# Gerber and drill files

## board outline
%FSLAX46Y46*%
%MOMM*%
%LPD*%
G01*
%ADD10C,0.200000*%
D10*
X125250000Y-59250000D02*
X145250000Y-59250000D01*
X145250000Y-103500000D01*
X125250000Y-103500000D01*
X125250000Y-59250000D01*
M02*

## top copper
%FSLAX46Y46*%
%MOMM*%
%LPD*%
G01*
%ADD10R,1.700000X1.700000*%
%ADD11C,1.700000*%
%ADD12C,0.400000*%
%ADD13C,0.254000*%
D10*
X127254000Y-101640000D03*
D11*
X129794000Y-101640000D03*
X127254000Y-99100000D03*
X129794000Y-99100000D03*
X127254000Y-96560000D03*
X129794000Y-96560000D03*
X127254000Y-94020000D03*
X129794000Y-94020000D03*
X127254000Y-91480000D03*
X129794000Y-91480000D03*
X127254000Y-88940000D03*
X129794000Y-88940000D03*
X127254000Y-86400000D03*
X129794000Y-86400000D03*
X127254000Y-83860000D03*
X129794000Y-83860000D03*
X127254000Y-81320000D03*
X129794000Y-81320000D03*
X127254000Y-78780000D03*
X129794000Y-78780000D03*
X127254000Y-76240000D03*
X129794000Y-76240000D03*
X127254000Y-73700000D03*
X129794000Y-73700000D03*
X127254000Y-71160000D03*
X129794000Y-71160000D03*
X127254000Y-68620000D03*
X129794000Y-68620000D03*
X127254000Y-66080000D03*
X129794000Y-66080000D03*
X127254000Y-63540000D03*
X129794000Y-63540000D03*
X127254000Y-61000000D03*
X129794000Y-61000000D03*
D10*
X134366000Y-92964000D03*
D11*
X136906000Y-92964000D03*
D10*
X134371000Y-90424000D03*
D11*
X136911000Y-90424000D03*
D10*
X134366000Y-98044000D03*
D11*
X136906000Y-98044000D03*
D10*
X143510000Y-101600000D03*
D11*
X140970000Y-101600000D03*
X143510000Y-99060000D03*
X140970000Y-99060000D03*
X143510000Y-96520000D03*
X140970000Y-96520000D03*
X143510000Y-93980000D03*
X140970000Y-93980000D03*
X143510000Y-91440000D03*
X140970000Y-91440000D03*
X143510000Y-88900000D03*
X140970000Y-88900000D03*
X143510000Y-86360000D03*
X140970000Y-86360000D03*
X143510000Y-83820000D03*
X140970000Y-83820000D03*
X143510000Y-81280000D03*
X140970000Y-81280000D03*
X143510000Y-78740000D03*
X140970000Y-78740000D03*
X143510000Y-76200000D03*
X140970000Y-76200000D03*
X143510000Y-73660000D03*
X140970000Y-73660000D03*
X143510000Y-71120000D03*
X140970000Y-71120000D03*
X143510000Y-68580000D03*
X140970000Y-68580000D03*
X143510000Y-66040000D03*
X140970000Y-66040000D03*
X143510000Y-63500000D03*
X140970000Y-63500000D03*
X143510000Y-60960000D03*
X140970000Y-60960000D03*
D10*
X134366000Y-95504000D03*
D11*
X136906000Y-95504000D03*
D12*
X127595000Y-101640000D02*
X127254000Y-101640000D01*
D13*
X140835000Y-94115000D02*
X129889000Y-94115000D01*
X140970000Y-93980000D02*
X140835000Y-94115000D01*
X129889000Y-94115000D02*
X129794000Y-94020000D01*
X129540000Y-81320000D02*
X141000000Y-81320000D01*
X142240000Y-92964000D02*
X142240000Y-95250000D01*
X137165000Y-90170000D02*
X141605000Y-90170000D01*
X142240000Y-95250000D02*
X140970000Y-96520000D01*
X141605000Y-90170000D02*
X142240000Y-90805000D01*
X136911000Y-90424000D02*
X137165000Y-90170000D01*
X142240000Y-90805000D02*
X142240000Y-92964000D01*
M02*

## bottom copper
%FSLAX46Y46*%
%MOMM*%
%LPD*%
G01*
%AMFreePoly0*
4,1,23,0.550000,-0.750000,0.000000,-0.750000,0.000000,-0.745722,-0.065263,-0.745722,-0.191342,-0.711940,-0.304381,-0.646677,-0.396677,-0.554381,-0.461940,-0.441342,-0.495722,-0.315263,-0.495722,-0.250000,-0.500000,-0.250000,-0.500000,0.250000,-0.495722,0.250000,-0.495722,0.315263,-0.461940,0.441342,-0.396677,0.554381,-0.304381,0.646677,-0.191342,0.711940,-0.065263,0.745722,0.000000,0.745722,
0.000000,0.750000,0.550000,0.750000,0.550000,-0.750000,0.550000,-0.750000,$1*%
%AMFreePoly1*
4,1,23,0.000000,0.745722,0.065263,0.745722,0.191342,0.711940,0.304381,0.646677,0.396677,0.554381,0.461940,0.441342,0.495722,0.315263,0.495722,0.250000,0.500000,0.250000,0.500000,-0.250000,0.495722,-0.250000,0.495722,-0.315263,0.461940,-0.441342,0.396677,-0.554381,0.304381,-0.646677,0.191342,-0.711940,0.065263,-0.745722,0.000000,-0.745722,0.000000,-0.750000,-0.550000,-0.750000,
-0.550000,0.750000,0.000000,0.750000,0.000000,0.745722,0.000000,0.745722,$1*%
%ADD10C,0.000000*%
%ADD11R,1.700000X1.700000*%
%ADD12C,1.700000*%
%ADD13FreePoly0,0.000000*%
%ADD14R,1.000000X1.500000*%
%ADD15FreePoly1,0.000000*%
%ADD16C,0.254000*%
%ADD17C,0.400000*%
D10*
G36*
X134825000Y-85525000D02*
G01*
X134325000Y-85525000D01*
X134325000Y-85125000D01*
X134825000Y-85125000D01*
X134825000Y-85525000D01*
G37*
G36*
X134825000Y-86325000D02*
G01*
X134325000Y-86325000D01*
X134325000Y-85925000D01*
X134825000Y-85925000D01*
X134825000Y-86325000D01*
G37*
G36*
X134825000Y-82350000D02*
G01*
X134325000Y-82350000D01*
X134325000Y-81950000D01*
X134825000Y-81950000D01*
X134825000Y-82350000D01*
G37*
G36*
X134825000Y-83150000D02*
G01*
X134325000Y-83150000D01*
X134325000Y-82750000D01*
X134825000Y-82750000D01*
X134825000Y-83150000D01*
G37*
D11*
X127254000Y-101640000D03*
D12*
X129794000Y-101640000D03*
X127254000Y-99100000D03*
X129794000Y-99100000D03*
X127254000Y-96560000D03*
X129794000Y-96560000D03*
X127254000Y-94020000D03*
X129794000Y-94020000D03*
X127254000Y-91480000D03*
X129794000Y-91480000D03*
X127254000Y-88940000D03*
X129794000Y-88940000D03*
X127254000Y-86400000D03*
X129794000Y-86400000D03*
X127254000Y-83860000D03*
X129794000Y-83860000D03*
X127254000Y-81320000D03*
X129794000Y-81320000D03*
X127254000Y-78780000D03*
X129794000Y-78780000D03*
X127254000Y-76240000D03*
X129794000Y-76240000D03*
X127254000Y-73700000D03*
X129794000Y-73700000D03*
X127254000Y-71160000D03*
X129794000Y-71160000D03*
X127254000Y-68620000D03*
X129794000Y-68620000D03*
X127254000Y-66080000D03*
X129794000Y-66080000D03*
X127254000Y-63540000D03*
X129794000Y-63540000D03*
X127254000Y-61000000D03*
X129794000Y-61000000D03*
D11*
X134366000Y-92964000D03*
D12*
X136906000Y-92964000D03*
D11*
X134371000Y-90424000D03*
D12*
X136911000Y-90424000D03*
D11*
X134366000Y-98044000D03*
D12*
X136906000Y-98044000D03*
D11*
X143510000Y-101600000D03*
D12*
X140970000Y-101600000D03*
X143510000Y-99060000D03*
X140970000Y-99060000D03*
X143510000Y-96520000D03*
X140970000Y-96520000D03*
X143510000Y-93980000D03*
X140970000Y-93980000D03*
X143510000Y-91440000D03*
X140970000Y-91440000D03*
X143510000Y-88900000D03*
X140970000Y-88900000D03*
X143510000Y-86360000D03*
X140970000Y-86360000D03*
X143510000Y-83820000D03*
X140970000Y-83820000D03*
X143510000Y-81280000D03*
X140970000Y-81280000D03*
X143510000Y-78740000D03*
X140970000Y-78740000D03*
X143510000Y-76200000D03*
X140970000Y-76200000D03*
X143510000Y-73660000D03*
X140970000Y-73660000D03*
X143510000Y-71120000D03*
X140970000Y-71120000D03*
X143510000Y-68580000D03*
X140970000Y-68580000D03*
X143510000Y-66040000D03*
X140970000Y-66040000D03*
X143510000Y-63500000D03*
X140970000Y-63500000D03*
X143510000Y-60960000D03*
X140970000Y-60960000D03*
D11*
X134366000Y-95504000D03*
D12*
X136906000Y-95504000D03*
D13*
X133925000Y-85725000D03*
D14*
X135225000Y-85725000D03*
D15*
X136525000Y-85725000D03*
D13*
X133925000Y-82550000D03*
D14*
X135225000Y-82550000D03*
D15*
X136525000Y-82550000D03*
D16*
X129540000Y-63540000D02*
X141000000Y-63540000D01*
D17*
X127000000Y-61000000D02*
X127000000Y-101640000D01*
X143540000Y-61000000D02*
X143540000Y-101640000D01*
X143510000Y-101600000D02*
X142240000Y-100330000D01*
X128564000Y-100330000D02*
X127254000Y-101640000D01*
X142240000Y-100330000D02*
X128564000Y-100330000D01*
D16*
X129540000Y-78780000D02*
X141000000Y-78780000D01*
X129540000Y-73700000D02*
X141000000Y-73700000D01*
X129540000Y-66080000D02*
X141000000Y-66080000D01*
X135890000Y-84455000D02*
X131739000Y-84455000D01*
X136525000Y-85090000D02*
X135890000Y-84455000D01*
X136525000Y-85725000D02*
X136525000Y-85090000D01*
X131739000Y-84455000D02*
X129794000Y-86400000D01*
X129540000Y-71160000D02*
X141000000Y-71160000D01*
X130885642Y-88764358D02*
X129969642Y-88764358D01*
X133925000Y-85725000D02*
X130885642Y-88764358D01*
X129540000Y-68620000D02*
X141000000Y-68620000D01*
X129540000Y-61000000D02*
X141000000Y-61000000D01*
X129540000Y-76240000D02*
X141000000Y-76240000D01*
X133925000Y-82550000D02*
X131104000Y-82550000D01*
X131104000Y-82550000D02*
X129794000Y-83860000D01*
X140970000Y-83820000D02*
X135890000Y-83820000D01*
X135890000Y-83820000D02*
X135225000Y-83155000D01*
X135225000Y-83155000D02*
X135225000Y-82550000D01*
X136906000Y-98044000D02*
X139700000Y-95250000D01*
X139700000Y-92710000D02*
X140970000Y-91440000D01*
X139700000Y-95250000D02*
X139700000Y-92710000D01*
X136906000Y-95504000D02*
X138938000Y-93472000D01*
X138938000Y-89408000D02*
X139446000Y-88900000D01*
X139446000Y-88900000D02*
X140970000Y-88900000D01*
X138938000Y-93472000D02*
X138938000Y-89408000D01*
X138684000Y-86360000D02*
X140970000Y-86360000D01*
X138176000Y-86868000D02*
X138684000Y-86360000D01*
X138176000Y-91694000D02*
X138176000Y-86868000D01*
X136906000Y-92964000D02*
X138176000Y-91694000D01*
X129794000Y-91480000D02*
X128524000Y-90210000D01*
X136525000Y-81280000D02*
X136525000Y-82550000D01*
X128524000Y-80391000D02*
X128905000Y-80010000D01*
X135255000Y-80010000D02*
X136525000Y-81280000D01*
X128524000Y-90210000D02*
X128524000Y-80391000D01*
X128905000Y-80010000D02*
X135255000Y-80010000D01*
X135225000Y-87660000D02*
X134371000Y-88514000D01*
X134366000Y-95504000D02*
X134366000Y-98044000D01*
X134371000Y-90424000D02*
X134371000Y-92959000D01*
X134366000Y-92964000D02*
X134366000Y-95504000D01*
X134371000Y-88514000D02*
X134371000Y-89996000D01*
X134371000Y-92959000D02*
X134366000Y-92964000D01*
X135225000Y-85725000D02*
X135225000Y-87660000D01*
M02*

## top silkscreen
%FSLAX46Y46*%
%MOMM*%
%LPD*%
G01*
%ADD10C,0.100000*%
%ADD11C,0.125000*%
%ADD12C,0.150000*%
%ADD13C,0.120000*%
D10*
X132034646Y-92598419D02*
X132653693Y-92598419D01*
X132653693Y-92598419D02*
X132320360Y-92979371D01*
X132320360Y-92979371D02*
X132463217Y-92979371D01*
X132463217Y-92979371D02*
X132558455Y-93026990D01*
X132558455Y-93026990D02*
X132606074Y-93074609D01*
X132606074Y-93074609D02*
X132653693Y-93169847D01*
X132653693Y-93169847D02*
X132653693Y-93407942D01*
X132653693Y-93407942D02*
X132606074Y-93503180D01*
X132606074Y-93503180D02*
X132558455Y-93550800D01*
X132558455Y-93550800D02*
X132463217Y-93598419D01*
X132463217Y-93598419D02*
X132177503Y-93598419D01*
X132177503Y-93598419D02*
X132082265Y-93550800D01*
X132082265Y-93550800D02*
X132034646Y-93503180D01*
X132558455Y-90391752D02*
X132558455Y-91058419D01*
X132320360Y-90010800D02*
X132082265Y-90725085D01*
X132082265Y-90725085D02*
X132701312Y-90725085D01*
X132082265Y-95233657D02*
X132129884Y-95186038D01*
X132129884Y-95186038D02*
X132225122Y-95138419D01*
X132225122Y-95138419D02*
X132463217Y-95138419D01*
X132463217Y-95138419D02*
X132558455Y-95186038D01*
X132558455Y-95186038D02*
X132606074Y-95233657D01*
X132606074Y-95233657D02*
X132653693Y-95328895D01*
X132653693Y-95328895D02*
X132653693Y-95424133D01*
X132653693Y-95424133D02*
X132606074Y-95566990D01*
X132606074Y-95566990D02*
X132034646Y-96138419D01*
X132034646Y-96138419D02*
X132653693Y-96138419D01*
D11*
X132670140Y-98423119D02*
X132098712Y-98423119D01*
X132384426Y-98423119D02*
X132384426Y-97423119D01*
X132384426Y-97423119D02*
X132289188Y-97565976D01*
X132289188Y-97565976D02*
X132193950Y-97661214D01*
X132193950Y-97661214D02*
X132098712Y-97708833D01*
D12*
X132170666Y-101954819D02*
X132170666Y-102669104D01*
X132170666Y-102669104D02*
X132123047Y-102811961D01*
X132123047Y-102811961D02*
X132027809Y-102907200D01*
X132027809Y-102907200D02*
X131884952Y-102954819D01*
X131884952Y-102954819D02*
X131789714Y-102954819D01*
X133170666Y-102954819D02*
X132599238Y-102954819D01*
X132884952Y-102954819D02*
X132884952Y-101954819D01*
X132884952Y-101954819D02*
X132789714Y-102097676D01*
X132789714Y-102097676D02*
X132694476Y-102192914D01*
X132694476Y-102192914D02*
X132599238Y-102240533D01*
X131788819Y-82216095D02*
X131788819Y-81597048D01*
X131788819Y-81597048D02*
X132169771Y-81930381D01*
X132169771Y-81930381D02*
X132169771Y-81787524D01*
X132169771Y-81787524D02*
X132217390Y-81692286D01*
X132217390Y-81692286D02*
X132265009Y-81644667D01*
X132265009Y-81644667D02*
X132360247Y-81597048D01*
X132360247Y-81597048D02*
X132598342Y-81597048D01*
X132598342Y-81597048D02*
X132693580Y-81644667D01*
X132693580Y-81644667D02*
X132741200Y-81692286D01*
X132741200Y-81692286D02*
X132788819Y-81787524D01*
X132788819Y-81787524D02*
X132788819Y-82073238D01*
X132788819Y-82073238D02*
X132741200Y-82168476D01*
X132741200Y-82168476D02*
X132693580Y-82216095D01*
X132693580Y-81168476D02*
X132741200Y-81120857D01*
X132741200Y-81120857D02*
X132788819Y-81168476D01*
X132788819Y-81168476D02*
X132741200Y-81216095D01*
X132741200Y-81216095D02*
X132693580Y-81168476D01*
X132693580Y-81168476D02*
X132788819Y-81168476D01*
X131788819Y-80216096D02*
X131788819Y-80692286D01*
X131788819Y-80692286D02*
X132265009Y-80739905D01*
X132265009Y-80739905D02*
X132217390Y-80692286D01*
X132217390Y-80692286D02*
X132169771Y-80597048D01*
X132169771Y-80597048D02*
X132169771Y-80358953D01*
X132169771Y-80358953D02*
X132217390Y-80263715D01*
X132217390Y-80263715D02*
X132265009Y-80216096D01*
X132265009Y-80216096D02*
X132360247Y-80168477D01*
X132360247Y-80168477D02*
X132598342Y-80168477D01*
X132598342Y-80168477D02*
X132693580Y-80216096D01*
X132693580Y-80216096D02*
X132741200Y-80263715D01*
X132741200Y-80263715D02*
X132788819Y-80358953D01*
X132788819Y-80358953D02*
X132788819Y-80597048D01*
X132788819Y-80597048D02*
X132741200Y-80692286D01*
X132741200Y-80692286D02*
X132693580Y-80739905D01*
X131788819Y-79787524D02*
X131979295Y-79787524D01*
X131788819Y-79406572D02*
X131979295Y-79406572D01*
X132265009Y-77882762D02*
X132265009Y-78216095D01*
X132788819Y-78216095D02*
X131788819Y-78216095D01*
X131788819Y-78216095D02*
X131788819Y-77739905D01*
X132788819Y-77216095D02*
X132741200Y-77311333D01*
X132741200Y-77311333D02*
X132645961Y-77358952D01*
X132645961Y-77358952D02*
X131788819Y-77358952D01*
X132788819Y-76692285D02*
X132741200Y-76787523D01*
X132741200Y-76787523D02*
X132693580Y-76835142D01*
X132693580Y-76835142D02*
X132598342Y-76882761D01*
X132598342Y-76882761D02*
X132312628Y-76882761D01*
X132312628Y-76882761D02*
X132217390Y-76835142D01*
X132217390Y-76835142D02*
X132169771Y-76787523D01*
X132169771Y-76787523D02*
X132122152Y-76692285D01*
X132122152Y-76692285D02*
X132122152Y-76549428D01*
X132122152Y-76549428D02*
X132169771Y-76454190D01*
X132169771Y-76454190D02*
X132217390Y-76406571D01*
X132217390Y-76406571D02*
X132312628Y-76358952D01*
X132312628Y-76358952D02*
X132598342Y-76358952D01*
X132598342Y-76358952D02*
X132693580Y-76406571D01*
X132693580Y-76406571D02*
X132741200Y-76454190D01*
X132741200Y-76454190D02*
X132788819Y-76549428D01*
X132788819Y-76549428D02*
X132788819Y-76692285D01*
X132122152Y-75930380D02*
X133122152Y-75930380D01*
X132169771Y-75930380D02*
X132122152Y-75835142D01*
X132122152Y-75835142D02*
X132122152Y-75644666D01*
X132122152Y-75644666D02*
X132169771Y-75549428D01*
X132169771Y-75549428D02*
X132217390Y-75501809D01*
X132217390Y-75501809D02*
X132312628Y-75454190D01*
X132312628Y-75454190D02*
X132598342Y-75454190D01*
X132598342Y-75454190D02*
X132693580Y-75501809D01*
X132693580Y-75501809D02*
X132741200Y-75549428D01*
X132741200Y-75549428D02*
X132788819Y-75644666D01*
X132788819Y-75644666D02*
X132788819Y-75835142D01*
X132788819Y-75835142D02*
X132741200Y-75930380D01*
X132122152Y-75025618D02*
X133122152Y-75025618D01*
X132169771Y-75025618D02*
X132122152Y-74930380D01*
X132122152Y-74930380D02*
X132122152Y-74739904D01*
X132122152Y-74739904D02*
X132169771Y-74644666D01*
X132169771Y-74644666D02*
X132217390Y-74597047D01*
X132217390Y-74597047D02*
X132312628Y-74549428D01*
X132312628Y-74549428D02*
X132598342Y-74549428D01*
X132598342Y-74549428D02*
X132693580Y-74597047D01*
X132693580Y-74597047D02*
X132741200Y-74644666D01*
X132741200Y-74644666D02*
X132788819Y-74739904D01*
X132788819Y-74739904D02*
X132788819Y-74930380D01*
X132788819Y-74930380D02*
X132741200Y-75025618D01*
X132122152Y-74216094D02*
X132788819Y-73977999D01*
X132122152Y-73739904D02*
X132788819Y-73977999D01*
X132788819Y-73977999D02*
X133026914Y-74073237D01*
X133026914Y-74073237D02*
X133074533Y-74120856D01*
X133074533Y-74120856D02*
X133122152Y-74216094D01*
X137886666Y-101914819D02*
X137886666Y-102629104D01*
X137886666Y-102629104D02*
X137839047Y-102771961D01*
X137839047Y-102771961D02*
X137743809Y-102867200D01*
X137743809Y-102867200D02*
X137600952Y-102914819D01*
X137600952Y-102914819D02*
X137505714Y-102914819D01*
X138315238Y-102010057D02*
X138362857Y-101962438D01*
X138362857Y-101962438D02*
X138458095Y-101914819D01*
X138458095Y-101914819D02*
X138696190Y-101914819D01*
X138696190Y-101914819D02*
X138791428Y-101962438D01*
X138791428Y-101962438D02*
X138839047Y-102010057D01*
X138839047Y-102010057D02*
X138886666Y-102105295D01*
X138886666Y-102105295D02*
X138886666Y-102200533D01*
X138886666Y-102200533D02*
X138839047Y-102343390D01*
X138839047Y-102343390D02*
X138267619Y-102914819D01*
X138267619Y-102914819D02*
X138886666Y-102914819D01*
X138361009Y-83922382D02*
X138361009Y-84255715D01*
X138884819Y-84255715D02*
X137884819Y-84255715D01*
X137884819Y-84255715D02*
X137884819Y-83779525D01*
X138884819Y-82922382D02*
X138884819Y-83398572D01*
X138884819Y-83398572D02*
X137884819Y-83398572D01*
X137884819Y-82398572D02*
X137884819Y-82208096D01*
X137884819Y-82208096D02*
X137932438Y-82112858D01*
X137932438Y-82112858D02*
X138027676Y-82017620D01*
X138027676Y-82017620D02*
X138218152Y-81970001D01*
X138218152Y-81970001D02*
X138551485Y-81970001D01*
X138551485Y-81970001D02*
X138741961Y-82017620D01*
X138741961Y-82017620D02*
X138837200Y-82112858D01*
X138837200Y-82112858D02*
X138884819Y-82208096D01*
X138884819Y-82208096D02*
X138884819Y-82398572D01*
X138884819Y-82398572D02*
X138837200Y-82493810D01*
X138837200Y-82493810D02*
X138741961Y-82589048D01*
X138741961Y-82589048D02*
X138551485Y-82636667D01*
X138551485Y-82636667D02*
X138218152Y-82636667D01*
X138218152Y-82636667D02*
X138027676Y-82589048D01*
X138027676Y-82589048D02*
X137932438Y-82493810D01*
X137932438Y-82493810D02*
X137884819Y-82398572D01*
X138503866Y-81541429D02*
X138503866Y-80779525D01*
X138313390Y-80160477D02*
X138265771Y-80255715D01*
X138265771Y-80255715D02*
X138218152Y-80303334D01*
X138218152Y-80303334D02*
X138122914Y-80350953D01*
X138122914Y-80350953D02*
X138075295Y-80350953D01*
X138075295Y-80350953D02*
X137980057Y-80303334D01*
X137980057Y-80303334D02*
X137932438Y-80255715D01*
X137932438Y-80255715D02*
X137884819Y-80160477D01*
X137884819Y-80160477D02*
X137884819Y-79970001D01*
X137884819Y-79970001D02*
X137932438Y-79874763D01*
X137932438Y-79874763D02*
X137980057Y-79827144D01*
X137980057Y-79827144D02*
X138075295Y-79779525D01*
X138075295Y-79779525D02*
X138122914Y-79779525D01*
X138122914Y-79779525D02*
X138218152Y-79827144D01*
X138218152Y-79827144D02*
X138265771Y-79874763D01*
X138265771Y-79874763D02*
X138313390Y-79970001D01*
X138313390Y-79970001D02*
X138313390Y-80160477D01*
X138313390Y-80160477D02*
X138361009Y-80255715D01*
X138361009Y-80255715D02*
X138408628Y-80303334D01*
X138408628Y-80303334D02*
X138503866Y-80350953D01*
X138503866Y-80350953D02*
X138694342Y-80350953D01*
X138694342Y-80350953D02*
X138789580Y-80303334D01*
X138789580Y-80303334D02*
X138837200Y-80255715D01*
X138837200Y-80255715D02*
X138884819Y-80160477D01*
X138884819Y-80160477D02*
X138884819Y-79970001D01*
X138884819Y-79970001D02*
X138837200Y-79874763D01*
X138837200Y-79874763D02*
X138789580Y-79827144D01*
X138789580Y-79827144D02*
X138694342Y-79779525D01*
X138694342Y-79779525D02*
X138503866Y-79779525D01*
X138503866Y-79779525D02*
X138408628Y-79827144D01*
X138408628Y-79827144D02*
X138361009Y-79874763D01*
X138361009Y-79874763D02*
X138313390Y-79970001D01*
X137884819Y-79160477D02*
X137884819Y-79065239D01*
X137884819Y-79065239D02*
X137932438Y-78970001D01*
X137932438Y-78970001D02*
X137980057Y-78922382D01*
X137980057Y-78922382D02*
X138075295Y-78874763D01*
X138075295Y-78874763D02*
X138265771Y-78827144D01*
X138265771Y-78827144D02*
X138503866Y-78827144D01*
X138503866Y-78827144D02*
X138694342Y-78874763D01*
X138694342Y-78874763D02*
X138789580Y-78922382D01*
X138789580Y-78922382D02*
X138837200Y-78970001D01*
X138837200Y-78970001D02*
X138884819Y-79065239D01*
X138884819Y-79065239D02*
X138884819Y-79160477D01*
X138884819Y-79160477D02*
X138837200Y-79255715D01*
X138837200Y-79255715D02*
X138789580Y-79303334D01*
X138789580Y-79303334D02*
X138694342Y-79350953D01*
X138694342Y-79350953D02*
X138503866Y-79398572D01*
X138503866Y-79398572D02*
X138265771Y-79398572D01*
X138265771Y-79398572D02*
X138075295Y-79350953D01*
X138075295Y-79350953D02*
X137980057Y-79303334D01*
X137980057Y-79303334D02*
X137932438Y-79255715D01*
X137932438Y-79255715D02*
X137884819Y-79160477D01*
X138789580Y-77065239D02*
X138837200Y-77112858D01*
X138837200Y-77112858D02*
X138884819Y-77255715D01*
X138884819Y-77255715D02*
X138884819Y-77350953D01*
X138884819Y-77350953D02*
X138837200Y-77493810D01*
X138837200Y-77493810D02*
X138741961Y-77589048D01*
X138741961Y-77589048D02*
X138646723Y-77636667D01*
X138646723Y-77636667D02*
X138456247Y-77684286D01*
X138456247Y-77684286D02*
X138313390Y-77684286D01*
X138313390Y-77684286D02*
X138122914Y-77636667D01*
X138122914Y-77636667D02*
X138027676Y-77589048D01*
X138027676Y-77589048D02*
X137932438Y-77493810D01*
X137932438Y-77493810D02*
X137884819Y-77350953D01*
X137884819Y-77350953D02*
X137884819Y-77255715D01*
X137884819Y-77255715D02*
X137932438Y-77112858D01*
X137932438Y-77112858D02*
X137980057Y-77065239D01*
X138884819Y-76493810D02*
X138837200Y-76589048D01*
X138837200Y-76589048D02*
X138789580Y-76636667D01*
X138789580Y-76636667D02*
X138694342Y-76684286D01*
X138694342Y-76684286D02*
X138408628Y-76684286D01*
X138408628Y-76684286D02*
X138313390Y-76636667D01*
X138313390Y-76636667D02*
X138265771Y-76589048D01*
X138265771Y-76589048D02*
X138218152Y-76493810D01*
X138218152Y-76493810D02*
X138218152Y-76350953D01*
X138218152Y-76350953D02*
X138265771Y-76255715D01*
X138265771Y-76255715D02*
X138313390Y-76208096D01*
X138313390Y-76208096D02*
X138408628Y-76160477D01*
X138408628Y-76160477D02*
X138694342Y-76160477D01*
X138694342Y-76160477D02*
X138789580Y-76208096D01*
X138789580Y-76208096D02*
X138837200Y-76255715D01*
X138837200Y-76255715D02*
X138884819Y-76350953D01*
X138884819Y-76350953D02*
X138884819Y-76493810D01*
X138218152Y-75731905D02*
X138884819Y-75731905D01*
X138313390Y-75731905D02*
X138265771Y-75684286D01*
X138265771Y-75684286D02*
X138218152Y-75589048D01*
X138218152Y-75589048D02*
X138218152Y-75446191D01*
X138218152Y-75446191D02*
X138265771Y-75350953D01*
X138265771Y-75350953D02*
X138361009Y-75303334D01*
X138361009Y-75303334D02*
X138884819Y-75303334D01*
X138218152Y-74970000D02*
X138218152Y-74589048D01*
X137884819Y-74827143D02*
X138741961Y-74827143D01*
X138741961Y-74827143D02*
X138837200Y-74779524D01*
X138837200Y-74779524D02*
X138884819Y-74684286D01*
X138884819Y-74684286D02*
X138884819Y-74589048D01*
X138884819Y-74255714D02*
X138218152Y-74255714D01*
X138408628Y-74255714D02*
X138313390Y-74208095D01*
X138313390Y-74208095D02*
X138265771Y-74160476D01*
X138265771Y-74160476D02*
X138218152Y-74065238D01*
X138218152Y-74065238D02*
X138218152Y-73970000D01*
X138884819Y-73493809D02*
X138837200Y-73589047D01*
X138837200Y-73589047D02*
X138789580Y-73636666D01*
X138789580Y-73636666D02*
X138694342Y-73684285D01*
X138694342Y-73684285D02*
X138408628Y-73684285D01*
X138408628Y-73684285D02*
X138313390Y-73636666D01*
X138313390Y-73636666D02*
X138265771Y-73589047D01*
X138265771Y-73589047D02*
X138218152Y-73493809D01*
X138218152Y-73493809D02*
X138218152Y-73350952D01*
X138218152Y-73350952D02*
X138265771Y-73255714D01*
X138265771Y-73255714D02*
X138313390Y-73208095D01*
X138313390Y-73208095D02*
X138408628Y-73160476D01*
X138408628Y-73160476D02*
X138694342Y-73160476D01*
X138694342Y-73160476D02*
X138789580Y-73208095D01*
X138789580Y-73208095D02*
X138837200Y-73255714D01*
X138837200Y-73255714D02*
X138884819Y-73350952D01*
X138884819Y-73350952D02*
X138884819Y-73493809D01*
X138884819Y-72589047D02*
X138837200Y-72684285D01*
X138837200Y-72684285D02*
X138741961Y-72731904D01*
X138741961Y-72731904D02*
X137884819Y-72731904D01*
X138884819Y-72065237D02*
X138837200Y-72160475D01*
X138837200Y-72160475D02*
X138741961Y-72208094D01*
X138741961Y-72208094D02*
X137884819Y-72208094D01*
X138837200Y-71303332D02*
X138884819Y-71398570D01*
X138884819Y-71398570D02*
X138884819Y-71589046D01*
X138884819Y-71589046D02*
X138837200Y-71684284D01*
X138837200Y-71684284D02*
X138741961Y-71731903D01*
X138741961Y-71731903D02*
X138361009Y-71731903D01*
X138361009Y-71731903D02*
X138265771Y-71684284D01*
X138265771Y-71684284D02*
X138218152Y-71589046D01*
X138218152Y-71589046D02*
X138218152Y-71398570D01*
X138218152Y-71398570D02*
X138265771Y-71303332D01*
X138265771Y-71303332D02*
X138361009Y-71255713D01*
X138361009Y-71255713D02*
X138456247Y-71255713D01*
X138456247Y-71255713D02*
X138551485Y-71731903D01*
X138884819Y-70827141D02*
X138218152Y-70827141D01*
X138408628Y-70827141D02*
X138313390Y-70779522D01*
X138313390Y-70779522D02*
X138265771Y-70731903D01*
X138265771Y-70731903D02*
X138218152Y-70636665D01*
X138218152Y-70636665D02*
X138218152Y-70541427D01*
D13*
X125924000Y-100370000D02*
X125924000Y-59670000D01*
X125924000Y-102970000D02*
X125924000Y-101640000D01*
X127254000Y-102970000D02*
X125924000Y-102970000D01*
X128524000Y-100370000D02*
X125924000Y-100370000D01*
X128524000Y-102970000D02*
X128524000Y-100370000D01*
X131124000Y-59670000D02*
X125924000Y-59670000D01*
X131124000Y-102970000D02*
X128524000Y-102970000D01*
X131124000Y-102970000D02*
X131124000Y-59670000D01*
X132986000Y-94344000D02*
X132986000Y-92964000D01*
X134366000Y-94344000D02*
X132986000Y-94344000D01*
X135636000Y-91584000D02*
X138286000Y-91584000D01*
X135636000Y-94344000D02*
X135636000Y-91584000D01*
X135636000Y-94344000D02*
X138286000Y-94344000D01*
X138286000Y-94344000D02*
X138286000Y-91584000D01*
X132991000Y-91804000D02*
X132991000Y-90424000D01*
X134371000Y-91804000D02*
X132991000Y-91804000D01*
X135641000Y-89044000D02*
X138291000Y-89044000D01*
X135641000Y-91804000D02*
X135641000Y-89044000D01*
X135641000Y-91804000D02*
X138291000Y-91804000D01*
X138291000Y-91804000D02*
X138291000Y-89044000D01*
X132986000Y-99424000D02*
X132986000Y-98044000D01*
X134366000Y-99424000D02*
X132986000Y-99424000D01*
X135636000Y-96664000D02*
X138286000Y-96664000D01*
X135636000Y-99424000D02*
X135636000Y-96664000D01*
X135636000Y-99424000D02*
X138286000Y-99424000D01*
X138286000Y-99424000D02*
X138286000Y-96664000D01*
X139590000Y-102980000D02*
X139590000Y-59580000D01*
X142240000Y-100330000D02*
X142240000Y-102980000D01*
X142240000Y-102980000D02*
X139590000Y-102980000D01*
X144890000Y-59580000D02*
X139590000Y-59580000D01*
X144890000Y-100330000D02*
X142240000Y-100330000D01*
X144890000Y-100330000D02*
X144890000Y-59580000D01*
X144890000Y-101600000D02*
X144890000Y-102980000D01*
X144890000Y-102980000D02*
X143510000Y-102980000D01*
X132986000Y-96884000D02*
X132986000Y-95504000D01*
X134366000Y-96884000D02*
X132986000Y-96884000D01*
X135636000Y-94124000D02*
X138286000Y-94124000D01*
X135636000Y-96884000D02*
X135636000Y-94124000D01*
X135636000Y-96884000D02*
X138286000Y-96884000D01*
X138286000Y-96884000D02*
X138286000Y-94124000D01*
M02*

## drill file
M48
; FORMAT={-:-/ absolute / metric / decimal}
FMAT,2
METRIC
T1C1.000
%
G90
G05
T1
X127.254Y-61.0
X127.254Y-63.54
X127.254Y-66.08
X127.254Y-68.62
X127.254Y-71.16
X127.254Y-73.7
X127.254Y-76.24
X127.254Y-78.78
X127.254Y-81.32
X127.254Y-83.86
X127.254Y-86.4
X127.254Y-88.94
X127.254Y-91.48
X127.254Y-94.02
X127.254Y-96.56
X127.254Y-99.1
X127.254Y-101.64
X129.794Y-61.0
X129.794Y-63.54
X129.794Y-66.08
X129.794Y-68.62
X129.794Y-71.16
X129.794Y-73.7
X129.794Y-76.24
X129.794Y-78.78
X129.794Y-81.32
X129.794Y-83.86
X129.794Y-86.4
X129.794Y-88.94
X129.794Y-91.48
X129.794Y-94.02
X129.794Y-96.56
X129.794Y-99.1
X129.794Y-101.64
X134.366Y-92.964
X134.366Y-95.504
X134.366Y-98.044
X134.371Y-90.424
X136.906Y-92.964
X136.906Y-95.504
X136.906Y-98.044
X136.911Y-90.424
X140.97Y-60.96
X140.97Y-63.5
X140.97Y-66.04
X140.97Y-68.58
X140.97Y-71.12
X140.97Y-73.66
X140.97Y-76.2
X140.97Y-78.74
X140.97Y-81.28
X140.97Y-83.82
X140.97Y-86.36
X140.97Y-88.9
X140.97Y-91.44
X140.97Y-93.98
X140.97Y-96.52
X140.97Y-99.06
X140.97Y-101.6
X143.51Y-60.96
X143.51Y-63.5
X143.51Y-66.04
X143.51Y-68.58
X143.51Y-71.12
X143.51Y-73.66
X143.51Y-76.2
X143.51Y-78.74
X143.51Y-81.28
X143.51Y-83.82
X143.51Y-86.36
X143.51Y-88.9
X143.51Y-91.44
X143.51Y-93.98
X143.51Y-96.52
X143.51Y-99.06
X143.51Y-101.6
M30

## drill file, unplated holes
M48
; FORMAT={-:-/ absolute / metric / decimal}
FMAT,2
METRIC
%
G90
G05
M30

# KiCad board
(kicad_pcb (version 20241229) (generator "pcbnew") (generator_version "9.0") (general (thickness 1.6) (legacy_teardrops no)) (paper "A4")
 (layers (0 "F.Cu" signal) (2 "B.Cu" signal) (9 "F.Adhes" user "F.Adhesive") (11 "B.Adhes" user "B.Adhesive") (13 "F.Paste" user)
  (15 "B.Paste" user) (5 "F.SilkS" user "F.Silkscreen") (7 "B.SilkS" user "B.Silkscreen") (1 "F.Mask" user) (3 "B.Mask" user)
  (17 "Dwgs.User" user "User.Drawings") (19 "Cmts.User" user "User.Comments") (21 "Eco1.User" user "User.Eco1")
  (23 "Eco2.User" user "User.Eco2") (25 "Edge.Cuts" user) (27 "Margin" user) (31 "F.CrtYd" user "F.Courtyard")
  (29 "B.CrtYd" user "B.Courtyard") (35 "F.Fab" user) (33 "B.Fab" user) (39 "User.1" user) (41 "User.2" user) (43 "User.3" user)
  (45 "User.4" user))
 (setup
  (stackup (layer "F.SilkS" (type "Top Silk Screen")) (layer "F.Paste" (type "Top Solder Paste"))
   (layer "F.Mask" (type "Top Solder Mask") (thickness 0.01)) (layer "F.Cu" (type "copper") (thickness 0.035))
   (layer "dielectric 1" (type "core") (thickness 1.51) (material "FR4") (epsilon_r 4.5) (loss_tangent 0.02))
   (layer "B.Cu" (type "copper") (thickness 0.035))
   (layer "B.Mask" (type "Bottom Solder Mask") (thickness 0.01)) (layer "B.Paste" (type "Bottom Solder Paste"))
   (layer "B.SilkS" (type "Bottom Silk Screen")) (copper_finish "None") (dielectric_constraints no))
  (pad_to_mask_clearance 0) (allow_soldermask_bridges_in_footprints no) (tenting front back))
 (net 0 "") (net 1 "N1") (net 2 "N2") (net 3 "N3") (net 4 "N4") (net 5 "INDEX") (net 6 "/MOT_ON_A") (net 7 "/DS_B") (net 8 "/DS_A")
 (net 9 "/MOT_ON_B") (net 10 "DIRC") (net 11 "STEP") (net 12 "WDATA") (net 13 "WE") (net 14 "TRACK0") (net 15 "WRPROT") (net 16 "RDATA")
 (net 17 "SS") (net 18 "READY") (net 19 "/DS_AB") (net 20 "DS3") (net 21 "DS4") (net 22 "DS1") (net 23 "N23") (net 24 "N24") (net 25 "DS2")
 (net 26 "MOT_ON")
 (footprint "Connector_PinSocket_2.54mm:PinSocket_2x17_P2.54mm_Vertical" (layer "F.Cu") (at 127.254 101.64 180)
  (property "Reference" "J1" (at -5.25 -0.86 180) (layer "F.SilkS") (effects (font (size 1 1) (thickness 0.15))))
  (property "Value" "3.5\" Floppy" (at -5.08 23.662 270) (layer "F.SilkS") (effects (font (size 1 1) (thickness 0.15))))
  (fp_line (start 1.33 1.27) (end 1.33 41.97) (stroke (width 0.12) (type solid)) (layer "F.SilkS"))
  (fp_line (start 1.33 -1.33) (end 1.33 0) (stroke (width 0.12) (type solid)) (layer "F.SilkS"))
  (fp_line (start 0 -1.33) (end 1.33 -1.33) (stroke (width 0.12) (type solid)) (layer "F.SilkS"))
  (fp_line (start -1.27 1.27) (end 1.33 1.27) (stroke (width 0.12) (type solid)) (layer "F.SilkS"))
  (fp_line (start -1.27 -1.33) (end -1.27 1.27) (stroke (width 0.12) (type solid)) (layer "F.SilkS"))
  (fp_line (start -3.87 41.97) (end 1.33 41.97) (stroke (width 0.12) (type solid)) (layer "F.SilkS"))
  (fp_line (start -3.87 -1.33) (end -1.27 -1.33) (stroke (width 0.12) (type solid)) (layer "F.SilkS"))
  (fp_line (start -3.87 -1.33) (end -3.87 41.97) (stroke (width 0.12) (type solid)) (layer "F.SilkS"))
  (pad "1" thru_hole rect (at 0 0 180) (size 1.7 1.7) (drill 1) (layers "*.Cu" "*.Mask") (remove_unused_layers no) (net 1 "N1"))
  (pad "2" thru_hole circle (at -2.54 0 180) (size 1.7 1.7) (drill 1) (layers "*.Cu" "*.Mask") (remove_unused_layers no) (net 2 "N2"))
  (pad "3" thru_hole circle (at 0 2.54 180) (size 1.7 1.7) (drill 1) (layers "*.Cu" "*.Mask") (remove_unused_layers no) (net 1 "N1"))
  (pad "4" thru_hole circle (at -2.54 2.54 180) (size 1.7 1.7) (drill 1) (layers "*.Cu" "*.Mask") (remove_unused_layers no) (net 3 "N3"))
  (pad "5" thru_hole circle (at 0 5.08 180) (size 1.7 1.7) (drill 1) (layers "*.Cu" "*.Mask") (remove_unused_layers no) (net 1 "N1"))
  (pad "6" thru_hole circle (at -2.54 5.08 180) (size 1.7 1.7) (drill 1) (layers "*.Cu" "*.Mask") (remove_unused_layers no) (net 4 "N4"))
  (pad "7" thru_hole circle (at 0 7.62 180) (size 1.7 1.7) (drill 1) (layers "*.Cu" "*.Mask") (remove_unused_layers no) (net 1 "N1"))
  (pad "8" thru_hole circle (at -2.54 7.62 180) (size 1.7 1.7) (drill 1) (layers "*.Cu" "*.Mask") (remove_unused_layers no) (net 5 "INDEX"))
  (pad "9" thru_hole circle (at 0 10.16 180) (size 1.7 1.7) (drill 1) (layers "*.Cu" "*.Mask") (remove_unused_layers no) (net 1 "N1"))
  (pad "10" thru_hole circle (at -2.54 10.16 180) (size 1.7 1.7) (drill 1) (layers "*.Cu" "*.Mask") (remove_unused_layers no)
   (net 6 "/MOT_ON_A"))
  (pad "11" thru_hole circle (at 0 12.7 180) (size 1.7 1.7) (drill 1) (layers "*.Cu" "*.Mask") (remove_unused_layers no) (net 1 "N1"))
  (pad "12" thru_hole circle (at -2.54 12.7 180) (size 1.7 1.7) (drill 1) (layers "*.Cu" "*.Mask") (remove_unused_layers no) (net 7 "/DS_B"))
  (pad "13" thru_hole circle (at 0 15.24 180) (size 1.7 1.7) (drill 1) (layers "*.Cu" "*.Mask") (remove_unused_layers no) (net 1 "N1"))
  (pad "14" thru_hole circle (at -2.54 15.24 180) (size 1.7 1.7) (drill 1) (layers "*.Cu" "*.Mask") (remove_unused_layers no)
   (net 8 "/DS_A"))
  (pad "15" thru_hole circle (at 0 17.78 180) (size 1.7 1.7) (drill 1) (layers "*.Cu" "*.Mask") (remove_unused_layers no) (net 1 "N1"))
  (pad "16" thru_hole circle (at -2.54 17.78 180) (size 1.7 1.7) (drill 1) (layers "*.Cu" "*.Mask") (remove_unused_layers no)
   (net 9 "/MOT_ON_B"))
  (pad "17" thru_hole circle (at 0 20.32 180) (size 1.7 1.7) (drill 1) (layers "*.Cu" "*.Mask") (remove_unused_layers no) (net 1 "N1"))
  (pad "18" thru_hole circle (at -2.54 20.32 180) (size 1.7 1.7) (drill 1) (layers "*.Cu" "*.Mask") (remove_unused_layers no)
   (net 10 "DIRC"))
  (pad "19" thru_hole circle (at 0 22.86 180) (size 1.7 1.7) (drill 1) (layers "*.Cu" "*.Mask") (remove_unused_layers no) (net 1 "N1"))
  (pad "20" thru_hole circle (at -2.54 22.86 180) (size 1.7 1.7) (drill 1) (layers "*.Cu" "*.Mask") (remove_unused_layers no)
   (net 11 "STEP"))
  (pad "21" thru_hole circle (at 0 25.4 180) (size 1.7 1.7) (drill 1) (layers "*.Cu" "*.Mask") (remove_unused_layers no) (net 1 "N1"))
  (pad "22" thru_hole circle (at -2.54 25.4 180) (size 1.7 1.7) (drill 1) (layers "*.Cu" "*.Mask") (remove_unused_layers no)
   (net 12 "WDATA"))
  (pad "23" thru_hole circle (at 0 27.94 180) (size 1.7 1.7) (drill 1) (layers "*.Cu" "*.Mask") (remove_unused_layers no) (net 1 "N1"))
  (pad "24" thru_hole circle (at -2.54 27.94 180) (size 1.7 1.7) (drill 1) (layers "*.Cu" "*.Mask") (remove_unused_layers no) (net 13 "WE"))
  (pad "25" thru_hole circle (at 0 30.48 180) (size 1.7 1.7) (drill 1) (layers "*.Cu" "*.Mask") (remove_unused_layers no) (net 1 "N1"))
  (pad "26" thru_hole circle (at -2.54 30.48 180) (size 1.7 1.7) (drill 1) (layers "*.Cu" "*.Mask") (remove_unused_layers no)
   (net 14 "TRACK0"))
  (pad "27" thru_hole circle (at 0 33.02 180) (size 1.7 1.7) (drill 1) (layers "*.Cu" "*.Mask") (remove_unused_layers no) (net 1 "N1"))
  (pad "28" thru_hole circle (at -2.54 33.02 180) (size 1.7 1.7) (drill 1) (layers "*.Cu" "*.Mask") (remove_unused_layers no)
   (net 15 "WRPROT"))
  (pad "29" thru_hole circle (at 0 35.56 180) (size 1.7 1.7) (drill 1) (layers "*.Cu" "*.Mask") (remove_unused_layers no) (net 1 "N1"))
  (pad "30" thru_hole circle (at -2.54 35.56 180) (size 1.7 1.7) (drill 1) (layers "*.Cu" "*.Mask") (remove_unused_layers no)
   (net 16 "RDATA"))
  (pad "31" thru_hole circle (at 0 38.1 180) (size 1.7 1.7) (drill 1) (layers "*.Cu" "*.Mask") (remove_unused_layers no) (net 1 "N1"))
  (pad "32" thru_hole circle (at -2.54 38.1 180) (size 1.7 1.7) (drill 1) (layers "*.Cu" "*.Mask") (remove_unused_layers no) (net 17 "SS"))
  (pad "33" thru_hole circle (at 0 40.64 180) (size 1.7 1.7) (drill 1) (layers "*.Cu" "*.Mask") (remove_unused_layers no) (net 1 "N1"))
  (pad "34" thru_hole circle (at -2.54 40.64 180) (size 1.7 1.7) (drill 1) (layers "*.Cu" "*.Mask") (remove_unused_layers no)
   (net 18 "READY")))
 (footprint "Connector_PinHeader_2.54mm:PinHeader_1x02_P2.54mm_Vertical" (layer "F.Cu") (at 134.366 92.964 90)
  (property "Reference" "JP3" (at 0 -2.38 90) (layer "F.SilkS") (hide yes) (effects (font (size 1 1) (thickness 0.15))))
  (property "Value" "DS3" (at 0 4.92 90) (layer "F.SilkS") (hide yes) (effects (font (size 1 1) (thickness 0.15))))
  (fp_line (start -1.38 -1.38) (end 0 -1.38) (stroke (width 0.12) (type solid)) (layer "F.SilkS"))
  (fp_line (start -1.38 0) (end -1.38 -1.38) (stroke (width 0.12) (type solid)) (layer "F.SilkS"))
  (fp_line (start 1.38 1.27) (end 1.38 3.92) (stroke (width 0.12) (type solid)) (layer "F.SilkS"))
  (fp_line (start -1.38 1.27) (end 1.38 1.27) (stroke (width 0.12) (type solid)) (layer "F.SilkS"))
  (fp_line (start -1.38 1.27) (end -1.38 3.92) (stroke (width 0.12) (type solid)) (layer "F.SilkS"))
  (fp_line (start -1.38 3.92) (end 1.38 3.92) (stroke (width 0.12) (type solid)) (layer "F.SilkS"))
  (pad "1" thru_hole rect (at 0 0 90) (size 1.7 1.7) (drill 1) (layers "*.Cu" "*.Mask") (remove_unused_layers no) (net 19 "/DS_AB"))
  (pad "2" thru_hole circle (at 0 2.54 90) (size 1.7 1.7) (drill 1) (layers "*.Cu" "*.Mask") (remove_unused_layers no) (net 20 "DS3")))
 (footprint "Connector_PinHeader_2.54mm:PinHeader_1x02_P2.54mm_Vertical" (layer "F.Cu") (at 134.371 90.424 90)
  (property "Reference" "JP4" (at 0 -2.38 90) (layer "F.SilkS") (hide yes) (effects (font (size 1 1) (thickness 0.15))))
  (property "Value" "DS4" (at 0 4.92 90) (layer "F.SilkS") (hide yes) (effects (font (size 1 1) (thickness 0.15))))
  (fp_line (start -1.38 -1.38) (end 0 -1.38) (stroke (width 0.12) (type solid)) (layer "F.SilkS"))
  (fp_line (start -1.38 0) (end -1.38 -1.38) (stroke (width 0.12) (type solid)) (layer "F.SilkS"))
  (fp_line (start 1.38 1.27) (end 1.38 3.92) (stroke (width 0.12) (type solid)) (layer "F.SilkS"))
  (fp_line (start -1.38 1.27) (end 1.38 1.27) (stroke (width 0.12) (type solid)) (layer "F.SilkS"))
  (fp_line (start -1.38 1.27) (end -1.38 3.92) (stroke (width 0.12) (type solid)) (layer "F.SilkS"))
  (fp_line (start -1.38 3.92) (end 1.38 3.92) (stroke (width 0.12) (type solid)) (layer "F.SilkS"))
  (pad "1" thru_hole rect (at 0 0 90) (size 1.7 1.7) (drill 1) (layers "*.Cu" "*.Mask") (remove_unused_layers no) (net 19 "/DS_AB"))
  (pad "2" thru_hole circle (at 0 2.54 90) (size 1.7 1.7) (drill 1) (layers "*.Cu" "*.Mask") (remove_unused_layers no) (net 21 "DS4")))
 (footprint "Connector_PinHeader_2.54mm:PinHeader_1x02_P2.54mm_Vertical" (layer "F.Cu") (at 134.366 98.044 90)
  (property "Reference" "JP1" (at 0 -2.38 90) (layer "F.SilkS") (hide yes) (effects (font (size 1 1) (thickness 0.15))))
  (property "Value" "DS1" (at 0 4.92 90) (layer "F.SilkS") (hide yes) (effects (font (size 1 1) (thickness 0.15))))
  (fp_line (start -1.38 -1.38) (end 0 -1.38) (stroke (width 0.12) (type solid)) (layer "F.SilkS"))
  (fp_line (start -1.38 0) (end -1.38 -1.38) (stroke (width 0.12) (type solid)) (layer "F.SilkS"))
  (fp_line (start 1.38 1.27) (end 1.38 3.92) (stroke (width 0.12) (type solid)) (layer "F.SilkS"))
  (fp_line (start -1.38 1.27) (end 1.38 1.27) (stroke (width 0.12) (type solid)) (layer "F.SilkS"))
  (fp_line (start -1.38 1.27) (end -1.38 3.92) (stroke (width 0.12) (type solid)) (layer "F.SilkS"))
  (fp_line (start -1.38 3.92) (end 1.38 3.92) (stroke (width 0.12) (type solid)) (layer "F.SilkS"))
  (pad "1" thru_hole rect (at 0 0 90) (size 1.7 1.7) (drill 1) (layers "*.Cu" "*.Mask") (remove_unused_layers no) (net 19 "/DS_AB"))
  (pad "2" thru_hole circle (at 0 2.54 90) (size 1.7 1.7) (drill 1) (layers "*.Cu" "*.Mask") (remove_unused_layers no) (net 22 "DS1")))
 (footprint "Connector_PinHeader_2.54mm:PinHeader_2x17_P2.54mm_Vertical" (layer "F.Cu") (at 143.51 101.6 180)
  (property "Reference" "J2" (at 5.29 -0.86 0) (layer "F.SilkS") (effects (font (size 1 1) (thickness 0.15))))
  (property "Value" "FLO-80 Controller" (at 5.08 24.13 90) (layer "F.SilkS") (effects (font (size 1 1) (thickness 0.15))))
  (fp_line (start 3.92 -1.38) (end 3.92 42.02) (stroke (width 0.12) (type solid)) (layer "F.SilkS"))
  (fp_line (start 1.27 1.27) (end 1.27 -1.38) (stroke (width 0.12) (type solid)) (layer "F.SilkS"))
  (fp_line (start 1.27 -1.38) (end 3.92 -1.38) (stroke (width 0.12) (type solid)) (layer "F.SilkS"))
  (fp_line (start -1.38 42.02) (end 3.92 42.02) (stroke (width 0.12) (type solid)) (layer "F.SilkS"))
  (fp_line (start -1.38 1.27) (end 1.27 1.27) (stroke (width 0.12) (type solid)) (layer "F.SilkS"))
  (fp_line (start -1.38 1.27) (end -1.38 42.02) (stroke (width 0.12) (type solid)) (layer "F.SilkS"))
  (fp_line (start -1.38 0) (end -1.38 -1.38) (stroke (width 0.12) (type solid)) (layer "F.SilkS"))
  (fp_line (start -1.38 -1.38) (end 0 -1.38) (stroke (width 0.12) (type solid)) (layer "F.SilkS"))
  (pad "1" thru_hole rect (at 0 0 180) (size 1.7 1.7) (drill 1) (layers "*.Cu" "*.Mask") (remove_unused_layers no) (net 1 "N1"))
  (pad "2" thru_hole circle (at 2.54 0 180) (size 1.7 1.7) (drill 1) (layers "*.Cu" "*.Mask") (remove_unused_layers no) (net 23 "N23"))
  (pad "3" thru_hole circle (at 0 2.54 180) (size 1.7 1.7) (drill 1) (layers "*.Cu" "*.Mask") (remove_unused_layers no) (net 1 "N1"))
  (pad "4" thru_hole circle (at 2.54 2.54 180) (size 1.7 1.7) (drill 1) (layers "*.Cu" "*.Mask") (remove_unused_layers no) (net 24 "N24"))
  (pad "5" thru_hole circle (at 0 5.08 180) (size 1.7 1.7) (drill 1) (layers "*.Cu" "*.Mask") (remove_unused_layers no) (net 1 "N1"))
  (pad "6" thru_hole circle (at 2.54 5.08 180) (size 1.7 1.7) (drill 1) (layers "*.Cu" "*.Mask") (remove_unused_layers no) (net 21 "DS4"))
  (pad "7" thru_hole circle (at 0 7.62 180) (size 1.7 1.7) (drill 1) (layers "*.Cu" "*.Mask") (remove_unused_layers no) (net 1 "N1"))
  (pad "8" thru_hole circle (at 2.54 7.62 180) (size 1.7 1.7) (drill 1) (layers "*.Cu" "*.Mask") (remove_unused_layers no) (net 5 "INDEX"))
  (pad "9" thru_hole circle (at 0 10.16 180) (size 1.7 1.7) (drill 1) (layers "*.Cu" "*.Mask") (remove_unused_layers no) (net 1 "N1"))
  (pad "10" thru_hole circle (at 2.54 10.16 180) (size 1.7 1.7) (drill 1) (layers "*.Cu" "*.Mask") (remove_unused_layers no) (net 22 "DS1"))
  (pad "11" thru_hole circle (at 0 12.7 180) (size 1.7 1.7) (drill 1) (layers "*.Cu" "*.Mask") (remove_unused_layers no) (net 1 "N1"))
  (pad "12" thru_hole circle (at 2.54 12.7 180) (size 1.7 1.7) (drill 1) (layers "*.Cu" "*.Mask") (remove_unused_layers no) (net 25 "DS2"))
  (pad "13" thru_hole circle (at 0 15.24 180) (size 1.7 1.7) (drill 1) (layers "*.Cu" "*.Mask") (remove_unused_layers no) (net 1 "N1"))
  (pad "14" thru_hole circle (at 2.54 15.24 180) (size 1.7 1.7) (drill 1) (layers "*.Cu" "*.Mask") (remove_unused_layers no) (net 20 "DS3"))
  (pad "15" thru_hole circle (at 0 17.78 180) (size 1.7 1.7) (drill 1) (layers "*.Cu" "*.Mask") (remove_unused_layers no) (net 1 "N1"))
  (pad "16" thru_hole circle (at 2.54 17.78 180) (size 1.7 1.7) (drill 1) (layers "*.Cu" "*.Mask") (remove_unused_layers no)
   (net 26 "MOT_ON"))
  (pad "17" thru_hole circle (at 0 20.32 180) (size 1.7 1.7) (drill 1) (layers "*.Cu" "*.Mask") (remove_unused_layers no) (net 1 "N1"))
  (pad "18" thru_hole circle (at 2.54 20.32 180) (size 1.7 1.7) (drill 1) (layers "*.Cu" "*.Mask") (remove_unused_layers no) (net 10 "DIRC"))
  (pad "19" thru_hole circle (at 0 22.86 180) (size 1.7 1.7) (drill 1) (layers "*.Cu" "*.Mask") (remove_unused_layers no) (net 1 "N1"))
  (pad "20" thru_hole circle (at 2.54 22.86 180) (size 1.7 1.7) (drill 1) (layers "*.Cu" "*.Mask") (remove_unused_layers no) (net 11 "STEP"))
  (pad "21" thru_hole circle (at 0 25.4 180) (size 1.7 1.7) (drill 1) (layers "*.Cu" "*.Mask") (remove_unused_layers no) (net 1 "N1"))
  (pad "22" thru_hole circle (at 2.54 25.4 180) (size 1.7 1.7) (drill 1) (layers "*.Cu" "*.Mask") (remove_unused_layers no) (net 12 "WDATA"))
  (pad "23" thru_hole circle (at 0 27.94 180) (size 1.7 1.7) (drill 1) (layers "*.Cu" "*.Mask") (remove_unused_layers no) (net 1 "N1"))
  (pad "24" thru_hole circle (at 2.54 27.94 180) (size 1.7 1.7) (drill 1) (layers "*.Cu" "*.Mask") (remove_unused_layers no) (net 13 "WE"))
  (pad "25" thru_hole circle (at 0 30.48 180) (size 1.7 1.7) (drill 1) (layers "*.Cu" "*.Mask") (remove_unused_layers no) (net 1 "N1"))
  (pad "26" thru_hole circle (at 2.54 30.48 180) (size 1.7 1.7) (drill 1) (layers "*.Cu" "*.Mask") (remove_unused_layers no)
   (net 14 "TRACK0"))
  (pad "27" thru_hole circle (at 0 33.02 180) (size 1.7 1.7) (drill 1) (layers "*.Cu" "*.Mask") (remove_unused_layers no) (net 1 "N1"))
  (pad "28" thru_hole circle (at 2.54 33.02 180) (size 1.7 1.7) (drill 1) (layers "*.Cu" "*.Mask") (remove_unused_layers no)
   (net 15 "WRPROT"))
  (pad "29" thru_hole circle (at 0 35.56 180) (size 1.7 1.7) (drill 1) (layers "*.Cu" "*.Mask") (remove_unused_layers no) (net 1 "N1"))
  (pad "30" thru_hole circle (at 2.54 35.56 180) (size 1.7 1.7) (drill 1) (layers "*.Cu" "*.Mask") (remove_unused_layers no)
   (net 16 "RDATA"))
  (pad "31" thru_hole circle (at 0 38.1 180) (size 1.7 1.7) (drill 1) (layers "*.Cu" "*.Mask") (remove_unused_layers no) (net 1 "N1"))
  (pad "32" thru_hole circle (at 2.54 38.1 180) (size 1.7 1.7) (drill 1) (layers "*.Cu" "*.Mask") (remove_unused_layers no) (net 17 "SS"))
  (pad "33" thru_hole circle (at 0 40.64 180) (size 1.7 1.7) (drill 1) (layers "*.Cu" "*.Mask") (remove_unused_layers no) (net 1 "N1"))
  (pad "34" thru_hole circle (at 2.54 40.64 180) (size 1.7 1.7) (drill 1) (layers "*.Cu" "*.Mask") (remove_unused_layers no)
   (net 18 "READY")))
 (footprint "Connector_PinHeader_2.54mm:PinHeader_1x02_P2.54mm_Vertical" (layer "F.Cu") (at 134.366 95.504 90)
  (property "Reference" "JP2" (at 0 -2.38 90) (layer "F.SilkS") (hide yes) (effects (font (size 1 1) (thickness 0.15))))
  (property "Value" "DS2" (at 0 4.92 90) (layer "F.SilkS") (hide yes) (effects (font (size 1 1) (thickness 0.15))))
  (fp_line (start -1.38 -1.38) (end 0 -1.38) (stroke (width 0.12) (type solid)) (layer "F.SilkS"))
  (fp_line (start -1.38 0) (end -1.38 -1.38) (stroke (width 0.12) (type solid)) (layer "F.SilkS"))
  (fp_line (start 1.38 1.27) (end 1.38 3.92) (stroke (width 0.12) (type solid)) (layer "F.SilkS"))
  (fp_line (start -1.38 1.27) (end 1.38 1.27) (stroke (width 0.12) (type solid)) (layer "F.SilkS"))
  (fp_line (start -1.38 1.27) (end -1.38 3.92) (stroke (width 0.12) (type solid)) (layer "F.SilkS"))
  (fp_line (start -1.38 3.92) (end 1.38 3.92) (stroke (width 0.12) (type solid)) (layer "F.SilkS"))
  (pad "1" thru_hole rect (at 0 0 90) (size 1.7 1.7) (drill 1) (layers "*.Cu" "*.Mask") (remove_unused_layers no) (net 19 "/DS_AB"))
  (pad "2" thru_hole circle (at 0 2.54 90) (size 1.7 1.7) (drill 1) (layers "*.Cu" "*.Mask") (remove_unused_layers no) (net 25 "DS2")))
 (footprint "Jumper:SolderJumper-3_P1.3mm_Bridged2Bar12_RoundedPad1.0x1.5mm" (layer "B.Cu") (at 135.225 85.725)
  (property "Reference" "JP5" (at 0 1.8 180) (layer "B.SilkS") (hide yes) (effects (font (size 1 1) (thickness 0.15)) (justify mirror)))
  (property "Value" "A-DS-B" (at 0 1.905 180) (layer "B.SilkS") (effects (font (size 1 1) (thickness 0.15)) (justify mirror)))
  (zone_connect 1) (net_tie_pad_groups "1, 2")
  (fp_poly (pts (xy -0.9 -0.2) (xy -0.4 -0.2) (xy -0.4 -0.6) (xy -0.9 -0.6)) (stroke (width 0) (type solid)) (fill yes) (layer "B.Cu"))
  (fp_poly (pts (xy -0.9 0.6) (xy -0.4 0.6) (xy -0.4 0.2) (xy -0.9 0.2)) (stroke (width 0) (type solid)) (fill yes) (layer "B.Cu"))
  (pad "1" smd custom (at -1.3 0) (size 1 0.5) (layers "B.Cu" "B.Mask") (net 7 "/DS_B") (zone_connect 2) (thermal_bridge_angle 45)
   (options (clearance outline) (anchor rect)) (primitives))
  (pad "2" smd rect (at 0 0) (size 1 1.5) (layers "B.Cu" "B.Mask") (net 19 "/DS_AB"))
  (pad "3" smd custom (at 1.3 0) (size 1 0.5) (layers "B.Cu" "B.Mask") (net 8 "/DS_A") (zone_connect 2) (thermal_bridge_angle 45)
   (options (clearance outline) (anchor rect)) (primitives)))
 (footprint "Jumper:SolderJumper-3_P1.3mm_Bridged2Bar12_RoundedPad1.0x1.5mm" (layer "B.Cu") (at 135.225 82.55)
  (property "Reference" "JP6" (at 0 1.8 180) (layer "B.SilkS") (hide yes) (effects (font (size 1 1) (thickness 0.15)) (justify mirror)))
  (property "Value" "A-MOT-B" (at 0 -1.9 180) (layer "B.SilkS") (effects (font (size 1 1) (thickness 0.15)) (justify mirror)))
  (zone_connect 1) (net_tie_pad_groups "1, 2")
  (fp_poly (pts (xy -0.9 -0.2) (xy -0.4 -0.2) (xy -0.4 -0.6) (xy -0.9 -0.6)) (stroke (width 0) (type solid)) (fill yes) (layer "B.Cu"))
  (fp_poly (pts (xy -0.9 0.6) (xy -0.4 0.6) (xy -0.4 0.2) (xy -0.9 0.2)) (stroke (width 0) (type solid)) (fill yes) (layer "B.Cu"))
  (pad "1" smd custom (at -1.3 0) (size 1 0.5) (layers "B.Cu" "B.Mask") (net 9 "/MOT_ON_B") (zone_connect 2) (thermal_bridge_angle 45)
   (options (clearance outline) (anchor rect)) (primitives))
  (pad "2" smd rect (at 0 0) (size 1 1.5) (layers "B.Cu" "B.Mask") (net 26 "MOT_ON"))
  (pad "3" smd custom (at 1.3 0) (size 1 0.5) (layers "B.Cu" "B.Mask") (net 6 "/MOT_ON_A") (zone_connect 2) (thermal_bridge_angle 45)
   (options (clearance outline) (anchor rect)) (primitives)))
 (gr_rect (start 125.25 59.25) (end 145.25 103.5) (stroke (width 0.2) (type solid)) (fill no) (layer "Edge.Cuts"))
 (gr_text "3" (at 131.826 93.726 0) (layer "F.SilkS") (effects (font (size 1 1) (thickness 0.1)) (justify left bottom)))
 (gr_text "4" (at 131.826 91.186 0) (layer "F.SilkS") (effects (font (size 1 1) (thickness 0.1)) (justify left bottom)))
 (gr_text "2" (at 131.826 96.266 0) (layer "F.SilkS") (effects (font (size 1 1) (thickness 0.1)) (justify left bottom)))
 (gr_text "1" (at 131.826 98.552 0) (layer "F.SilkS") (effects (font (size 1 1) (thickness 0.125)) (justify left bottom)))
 (segment (start 129.54 63.54) (end 141 63.54) (width 0.254) (layer "B.Cu") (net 17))
 (segment (start 127.595 101.64) (end 127.254 101.64) (width 0.4) (layer "F.Cu") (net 1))
 (segment (start 127 61) (end 127 101.64) (width 0.4) (layer "B.Cu") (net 1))
 (segment (start 143.54 61) (end 143.54 101.64) (width 0.4) (layer "B.Cu") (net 1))
 (segment (start 143.51 101.6) (end 142.24 100.33) (width 0.4) (layer "B.Cu") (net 1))
 (segment (start 128.564 100.33) (end 127.254 101.64) (width 0.4) (layer "B.Cu") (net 1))
 (segment (start 142.24 100.33) (end 128.564 100.33) (width 0.4) (layer "B.Cu") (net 1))
 (segment (start 129.54 78.78) (end 141 78.78) (width 0.254) (layer "B.Cu") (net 11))
 (segment (start 129.54 73.7) (end 141 73.7) (width 0.254) (layer "B.Cu") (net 13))
 (segment (start 129.54 66.08) (end 141 66.08) (width 0.254) (layer "B.Cu") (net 16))
 (segment (start 140.835 94.115) (end 129.889 94.115) (width 0.254) (layer "F.Cu") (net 5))
 (segment (start 140.97 93.98) (end 140.835 94.115) (width 0.254) (layer "F.Cu") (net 5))
 (segment (start 129.889 94.115) (end 129.794 94.02) (width 0.254) (layer "F.Cu") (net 5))
 (segment (start 135.89 84.455) (end 131.739 84.455) (width 0.254) (layer "B.Cu") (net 8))
 (segment (start 136.525 85.09) (end 135.89 84.455) (width 0.254) (layer "B.Cu") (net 8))
 (segment (start 136.525 85.725) (end 136.525 85.09) (width 0.254) (layer "B.Cu") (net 8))
 (segment (start 131.739 84.455) (end 129.794 86.4) (width 0.254) (layer "B.Cu") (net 8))
 (segment (start 129.54 71.16) (end 141 71.16) (width 0.254) (layer "B.Cu") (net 14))
 (segment (start 129.54 81.32) (end 141 81.32) (width 0.254) (layer "F.Cu") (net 10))
 (segment (start 130.885642 88.764358) (end 129.969642 88.764358) (width 0.254) (layer "B.Cu") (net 7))
 (segment (start 133.925 85.725) (end 130.885642 88.764358) (width 0.254) (layer "B.Cu") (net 7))
 (segment (start 129.54 68.62) (end 141 68.62) (width 0.254) (layer "B.Cu") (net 15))
 (segment (start 129.54 61) (end 141 61) (width 0.254) (layer "B.Cu") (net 18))
 (segment (start 129.54 76.24) (end 141 76.24) (width 0.254) (layer "B.Cu") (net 12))
 (segment (start 133.925 82.55) (end 131.104 82.55) (width 0.254) (layer "B.Cu") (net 9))
 (segment (start 131.104 82.55) (end 129.794 83.86) (width 0.254) (layer "B.Cu") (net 9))
 (segment (start 140.97 83.82) (end 135.89 83.82) (width 0.254) (layer "B.Cu") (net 26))
 (segment (start 135.89 83.82) (end 135.225 83.155) (width 0.254) (layer "B.Cu") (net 26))
 (segment (start 135.225 83.155) (end 135.225 82.55) (width 0.254) (layer "B.Cu") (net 26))
 (segment (start 136.906 98.044) (end 139.7 95.25) (width 0.254) (layer "B.Cu") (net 22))
 (segment (start 139.7 92.71) (end 140.97 91.44) (width 0.254) (layer "B.Cu") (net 22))
 (segment (start 139.7 95.25) (end 139.7 92.71) (width 0.254) (layer "B.Cu") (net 22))
 (segment (start 136.906 95.504) (end 138.938 93.472) (width 0.254) (layer "B.Cu") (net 25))
 (segment (start 138.938 89.408) (end 139.446 88.9) (width 0.254) (layer "B.Cu") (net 25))
 (segment (start 139.446 88.9) (end 140.97 88.9) (width 0.254) (layer "B.Cu") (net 25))
 (segment (start 138.938 93.472) (end 138.938 89.408) (width 0.254) (layer "B.Cu") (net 25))
 (segment (start 142.24 92.964) (end 142.24 95.25) (width 0.254) (layer "F.Cu") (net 21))
 (segment (start 137.165 90.17) (end 141.605 90.17) (width 0.254) (layer "F.Cu") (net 21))
 (segment (start 142.24 95.25) (end 140.97 96.52) (width 0.254) (layer "F.Cu") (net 21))
 (segment (start 141.605 90.17) (end 142.24 90.805) (width 0.254) (layer "F.Cu") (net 21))
 (segment (start 136.911 90.424) (end 137.165 90.17) (width 0.254) (layer "F.Cu") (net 21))
 (segment (start 142.24 90.805) (end 142.24 92.964) (width 0.254) (layer "F.Cu") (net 21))
 (segment (start 138.684 86.36) (end 140.97 86.36) (width 0.254) (layer "B.Cu") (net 20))
 (segment (start 138.176 86.868) (end 138.684 86.36) (width 0.254) (layer "B.Cu") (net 20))
 (segment (start 138.176 91.694) (end 138.176 86.868) (width 0.254) (layer "B.Cu") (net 20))
 (segment (start 136.906 92.964) (end 138.176 91.694) (width 0.254) (layer "B.Cu") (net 20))
 (segment (start 129.794 91.48) (end 128.524 90.21) (width 0.254) (layer "B.Cu") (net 6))
 (segment (start 136.525 81.28) (end 136.525 82.55) (width 0.254) (layer "B.Cu") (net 6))
 (segment (start 128.524 80.391) (end 128.905 80.01) (width 0.254) (layer "B.Cu") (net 6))
 (segment (start 135.255 80.01) (end 136.525 81.28) (width 0.254) (layer "B.Cu") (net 6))
 (segment (start 128.524 90.21) (end 128.524 80.391) (width 0.254) (layer "B.Cu") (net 6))
 (segment (start 128.905 80.01) (end 135.255 80.01) (width 0.254) (layer "B.Cu") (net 6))
 (segment (start 135.225 87.66) (end 134.371 88.514) (width 0.254) (layer "B.Cu") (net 19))
 (segment (start 134.366 95.504) (end 134.366 98.044) (width 0.254) (layer "B.Cu") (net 19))
 (segment (start 134.371 90.424) (end 134.371 92.959) (width 0.254) (layer "B.Cu") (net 19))
 (segment (start 134.366 92.964) (end 134.366 95.504) (width 0.254) (layer "B.Cu") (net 19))
 (segment (start 134.371 88.514) (end 134.371 89.996) (width 0.254) (layer "B.Cu") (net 19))
 (segment (start 134.371 92.959) (end 134.366 92.964) (width 0.254) (layer "B.Cu") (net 19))
 (segment (start 135.225 85.725) (end 135.225 87.66) (width 0.254) (layer "B.Cu") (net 19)))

